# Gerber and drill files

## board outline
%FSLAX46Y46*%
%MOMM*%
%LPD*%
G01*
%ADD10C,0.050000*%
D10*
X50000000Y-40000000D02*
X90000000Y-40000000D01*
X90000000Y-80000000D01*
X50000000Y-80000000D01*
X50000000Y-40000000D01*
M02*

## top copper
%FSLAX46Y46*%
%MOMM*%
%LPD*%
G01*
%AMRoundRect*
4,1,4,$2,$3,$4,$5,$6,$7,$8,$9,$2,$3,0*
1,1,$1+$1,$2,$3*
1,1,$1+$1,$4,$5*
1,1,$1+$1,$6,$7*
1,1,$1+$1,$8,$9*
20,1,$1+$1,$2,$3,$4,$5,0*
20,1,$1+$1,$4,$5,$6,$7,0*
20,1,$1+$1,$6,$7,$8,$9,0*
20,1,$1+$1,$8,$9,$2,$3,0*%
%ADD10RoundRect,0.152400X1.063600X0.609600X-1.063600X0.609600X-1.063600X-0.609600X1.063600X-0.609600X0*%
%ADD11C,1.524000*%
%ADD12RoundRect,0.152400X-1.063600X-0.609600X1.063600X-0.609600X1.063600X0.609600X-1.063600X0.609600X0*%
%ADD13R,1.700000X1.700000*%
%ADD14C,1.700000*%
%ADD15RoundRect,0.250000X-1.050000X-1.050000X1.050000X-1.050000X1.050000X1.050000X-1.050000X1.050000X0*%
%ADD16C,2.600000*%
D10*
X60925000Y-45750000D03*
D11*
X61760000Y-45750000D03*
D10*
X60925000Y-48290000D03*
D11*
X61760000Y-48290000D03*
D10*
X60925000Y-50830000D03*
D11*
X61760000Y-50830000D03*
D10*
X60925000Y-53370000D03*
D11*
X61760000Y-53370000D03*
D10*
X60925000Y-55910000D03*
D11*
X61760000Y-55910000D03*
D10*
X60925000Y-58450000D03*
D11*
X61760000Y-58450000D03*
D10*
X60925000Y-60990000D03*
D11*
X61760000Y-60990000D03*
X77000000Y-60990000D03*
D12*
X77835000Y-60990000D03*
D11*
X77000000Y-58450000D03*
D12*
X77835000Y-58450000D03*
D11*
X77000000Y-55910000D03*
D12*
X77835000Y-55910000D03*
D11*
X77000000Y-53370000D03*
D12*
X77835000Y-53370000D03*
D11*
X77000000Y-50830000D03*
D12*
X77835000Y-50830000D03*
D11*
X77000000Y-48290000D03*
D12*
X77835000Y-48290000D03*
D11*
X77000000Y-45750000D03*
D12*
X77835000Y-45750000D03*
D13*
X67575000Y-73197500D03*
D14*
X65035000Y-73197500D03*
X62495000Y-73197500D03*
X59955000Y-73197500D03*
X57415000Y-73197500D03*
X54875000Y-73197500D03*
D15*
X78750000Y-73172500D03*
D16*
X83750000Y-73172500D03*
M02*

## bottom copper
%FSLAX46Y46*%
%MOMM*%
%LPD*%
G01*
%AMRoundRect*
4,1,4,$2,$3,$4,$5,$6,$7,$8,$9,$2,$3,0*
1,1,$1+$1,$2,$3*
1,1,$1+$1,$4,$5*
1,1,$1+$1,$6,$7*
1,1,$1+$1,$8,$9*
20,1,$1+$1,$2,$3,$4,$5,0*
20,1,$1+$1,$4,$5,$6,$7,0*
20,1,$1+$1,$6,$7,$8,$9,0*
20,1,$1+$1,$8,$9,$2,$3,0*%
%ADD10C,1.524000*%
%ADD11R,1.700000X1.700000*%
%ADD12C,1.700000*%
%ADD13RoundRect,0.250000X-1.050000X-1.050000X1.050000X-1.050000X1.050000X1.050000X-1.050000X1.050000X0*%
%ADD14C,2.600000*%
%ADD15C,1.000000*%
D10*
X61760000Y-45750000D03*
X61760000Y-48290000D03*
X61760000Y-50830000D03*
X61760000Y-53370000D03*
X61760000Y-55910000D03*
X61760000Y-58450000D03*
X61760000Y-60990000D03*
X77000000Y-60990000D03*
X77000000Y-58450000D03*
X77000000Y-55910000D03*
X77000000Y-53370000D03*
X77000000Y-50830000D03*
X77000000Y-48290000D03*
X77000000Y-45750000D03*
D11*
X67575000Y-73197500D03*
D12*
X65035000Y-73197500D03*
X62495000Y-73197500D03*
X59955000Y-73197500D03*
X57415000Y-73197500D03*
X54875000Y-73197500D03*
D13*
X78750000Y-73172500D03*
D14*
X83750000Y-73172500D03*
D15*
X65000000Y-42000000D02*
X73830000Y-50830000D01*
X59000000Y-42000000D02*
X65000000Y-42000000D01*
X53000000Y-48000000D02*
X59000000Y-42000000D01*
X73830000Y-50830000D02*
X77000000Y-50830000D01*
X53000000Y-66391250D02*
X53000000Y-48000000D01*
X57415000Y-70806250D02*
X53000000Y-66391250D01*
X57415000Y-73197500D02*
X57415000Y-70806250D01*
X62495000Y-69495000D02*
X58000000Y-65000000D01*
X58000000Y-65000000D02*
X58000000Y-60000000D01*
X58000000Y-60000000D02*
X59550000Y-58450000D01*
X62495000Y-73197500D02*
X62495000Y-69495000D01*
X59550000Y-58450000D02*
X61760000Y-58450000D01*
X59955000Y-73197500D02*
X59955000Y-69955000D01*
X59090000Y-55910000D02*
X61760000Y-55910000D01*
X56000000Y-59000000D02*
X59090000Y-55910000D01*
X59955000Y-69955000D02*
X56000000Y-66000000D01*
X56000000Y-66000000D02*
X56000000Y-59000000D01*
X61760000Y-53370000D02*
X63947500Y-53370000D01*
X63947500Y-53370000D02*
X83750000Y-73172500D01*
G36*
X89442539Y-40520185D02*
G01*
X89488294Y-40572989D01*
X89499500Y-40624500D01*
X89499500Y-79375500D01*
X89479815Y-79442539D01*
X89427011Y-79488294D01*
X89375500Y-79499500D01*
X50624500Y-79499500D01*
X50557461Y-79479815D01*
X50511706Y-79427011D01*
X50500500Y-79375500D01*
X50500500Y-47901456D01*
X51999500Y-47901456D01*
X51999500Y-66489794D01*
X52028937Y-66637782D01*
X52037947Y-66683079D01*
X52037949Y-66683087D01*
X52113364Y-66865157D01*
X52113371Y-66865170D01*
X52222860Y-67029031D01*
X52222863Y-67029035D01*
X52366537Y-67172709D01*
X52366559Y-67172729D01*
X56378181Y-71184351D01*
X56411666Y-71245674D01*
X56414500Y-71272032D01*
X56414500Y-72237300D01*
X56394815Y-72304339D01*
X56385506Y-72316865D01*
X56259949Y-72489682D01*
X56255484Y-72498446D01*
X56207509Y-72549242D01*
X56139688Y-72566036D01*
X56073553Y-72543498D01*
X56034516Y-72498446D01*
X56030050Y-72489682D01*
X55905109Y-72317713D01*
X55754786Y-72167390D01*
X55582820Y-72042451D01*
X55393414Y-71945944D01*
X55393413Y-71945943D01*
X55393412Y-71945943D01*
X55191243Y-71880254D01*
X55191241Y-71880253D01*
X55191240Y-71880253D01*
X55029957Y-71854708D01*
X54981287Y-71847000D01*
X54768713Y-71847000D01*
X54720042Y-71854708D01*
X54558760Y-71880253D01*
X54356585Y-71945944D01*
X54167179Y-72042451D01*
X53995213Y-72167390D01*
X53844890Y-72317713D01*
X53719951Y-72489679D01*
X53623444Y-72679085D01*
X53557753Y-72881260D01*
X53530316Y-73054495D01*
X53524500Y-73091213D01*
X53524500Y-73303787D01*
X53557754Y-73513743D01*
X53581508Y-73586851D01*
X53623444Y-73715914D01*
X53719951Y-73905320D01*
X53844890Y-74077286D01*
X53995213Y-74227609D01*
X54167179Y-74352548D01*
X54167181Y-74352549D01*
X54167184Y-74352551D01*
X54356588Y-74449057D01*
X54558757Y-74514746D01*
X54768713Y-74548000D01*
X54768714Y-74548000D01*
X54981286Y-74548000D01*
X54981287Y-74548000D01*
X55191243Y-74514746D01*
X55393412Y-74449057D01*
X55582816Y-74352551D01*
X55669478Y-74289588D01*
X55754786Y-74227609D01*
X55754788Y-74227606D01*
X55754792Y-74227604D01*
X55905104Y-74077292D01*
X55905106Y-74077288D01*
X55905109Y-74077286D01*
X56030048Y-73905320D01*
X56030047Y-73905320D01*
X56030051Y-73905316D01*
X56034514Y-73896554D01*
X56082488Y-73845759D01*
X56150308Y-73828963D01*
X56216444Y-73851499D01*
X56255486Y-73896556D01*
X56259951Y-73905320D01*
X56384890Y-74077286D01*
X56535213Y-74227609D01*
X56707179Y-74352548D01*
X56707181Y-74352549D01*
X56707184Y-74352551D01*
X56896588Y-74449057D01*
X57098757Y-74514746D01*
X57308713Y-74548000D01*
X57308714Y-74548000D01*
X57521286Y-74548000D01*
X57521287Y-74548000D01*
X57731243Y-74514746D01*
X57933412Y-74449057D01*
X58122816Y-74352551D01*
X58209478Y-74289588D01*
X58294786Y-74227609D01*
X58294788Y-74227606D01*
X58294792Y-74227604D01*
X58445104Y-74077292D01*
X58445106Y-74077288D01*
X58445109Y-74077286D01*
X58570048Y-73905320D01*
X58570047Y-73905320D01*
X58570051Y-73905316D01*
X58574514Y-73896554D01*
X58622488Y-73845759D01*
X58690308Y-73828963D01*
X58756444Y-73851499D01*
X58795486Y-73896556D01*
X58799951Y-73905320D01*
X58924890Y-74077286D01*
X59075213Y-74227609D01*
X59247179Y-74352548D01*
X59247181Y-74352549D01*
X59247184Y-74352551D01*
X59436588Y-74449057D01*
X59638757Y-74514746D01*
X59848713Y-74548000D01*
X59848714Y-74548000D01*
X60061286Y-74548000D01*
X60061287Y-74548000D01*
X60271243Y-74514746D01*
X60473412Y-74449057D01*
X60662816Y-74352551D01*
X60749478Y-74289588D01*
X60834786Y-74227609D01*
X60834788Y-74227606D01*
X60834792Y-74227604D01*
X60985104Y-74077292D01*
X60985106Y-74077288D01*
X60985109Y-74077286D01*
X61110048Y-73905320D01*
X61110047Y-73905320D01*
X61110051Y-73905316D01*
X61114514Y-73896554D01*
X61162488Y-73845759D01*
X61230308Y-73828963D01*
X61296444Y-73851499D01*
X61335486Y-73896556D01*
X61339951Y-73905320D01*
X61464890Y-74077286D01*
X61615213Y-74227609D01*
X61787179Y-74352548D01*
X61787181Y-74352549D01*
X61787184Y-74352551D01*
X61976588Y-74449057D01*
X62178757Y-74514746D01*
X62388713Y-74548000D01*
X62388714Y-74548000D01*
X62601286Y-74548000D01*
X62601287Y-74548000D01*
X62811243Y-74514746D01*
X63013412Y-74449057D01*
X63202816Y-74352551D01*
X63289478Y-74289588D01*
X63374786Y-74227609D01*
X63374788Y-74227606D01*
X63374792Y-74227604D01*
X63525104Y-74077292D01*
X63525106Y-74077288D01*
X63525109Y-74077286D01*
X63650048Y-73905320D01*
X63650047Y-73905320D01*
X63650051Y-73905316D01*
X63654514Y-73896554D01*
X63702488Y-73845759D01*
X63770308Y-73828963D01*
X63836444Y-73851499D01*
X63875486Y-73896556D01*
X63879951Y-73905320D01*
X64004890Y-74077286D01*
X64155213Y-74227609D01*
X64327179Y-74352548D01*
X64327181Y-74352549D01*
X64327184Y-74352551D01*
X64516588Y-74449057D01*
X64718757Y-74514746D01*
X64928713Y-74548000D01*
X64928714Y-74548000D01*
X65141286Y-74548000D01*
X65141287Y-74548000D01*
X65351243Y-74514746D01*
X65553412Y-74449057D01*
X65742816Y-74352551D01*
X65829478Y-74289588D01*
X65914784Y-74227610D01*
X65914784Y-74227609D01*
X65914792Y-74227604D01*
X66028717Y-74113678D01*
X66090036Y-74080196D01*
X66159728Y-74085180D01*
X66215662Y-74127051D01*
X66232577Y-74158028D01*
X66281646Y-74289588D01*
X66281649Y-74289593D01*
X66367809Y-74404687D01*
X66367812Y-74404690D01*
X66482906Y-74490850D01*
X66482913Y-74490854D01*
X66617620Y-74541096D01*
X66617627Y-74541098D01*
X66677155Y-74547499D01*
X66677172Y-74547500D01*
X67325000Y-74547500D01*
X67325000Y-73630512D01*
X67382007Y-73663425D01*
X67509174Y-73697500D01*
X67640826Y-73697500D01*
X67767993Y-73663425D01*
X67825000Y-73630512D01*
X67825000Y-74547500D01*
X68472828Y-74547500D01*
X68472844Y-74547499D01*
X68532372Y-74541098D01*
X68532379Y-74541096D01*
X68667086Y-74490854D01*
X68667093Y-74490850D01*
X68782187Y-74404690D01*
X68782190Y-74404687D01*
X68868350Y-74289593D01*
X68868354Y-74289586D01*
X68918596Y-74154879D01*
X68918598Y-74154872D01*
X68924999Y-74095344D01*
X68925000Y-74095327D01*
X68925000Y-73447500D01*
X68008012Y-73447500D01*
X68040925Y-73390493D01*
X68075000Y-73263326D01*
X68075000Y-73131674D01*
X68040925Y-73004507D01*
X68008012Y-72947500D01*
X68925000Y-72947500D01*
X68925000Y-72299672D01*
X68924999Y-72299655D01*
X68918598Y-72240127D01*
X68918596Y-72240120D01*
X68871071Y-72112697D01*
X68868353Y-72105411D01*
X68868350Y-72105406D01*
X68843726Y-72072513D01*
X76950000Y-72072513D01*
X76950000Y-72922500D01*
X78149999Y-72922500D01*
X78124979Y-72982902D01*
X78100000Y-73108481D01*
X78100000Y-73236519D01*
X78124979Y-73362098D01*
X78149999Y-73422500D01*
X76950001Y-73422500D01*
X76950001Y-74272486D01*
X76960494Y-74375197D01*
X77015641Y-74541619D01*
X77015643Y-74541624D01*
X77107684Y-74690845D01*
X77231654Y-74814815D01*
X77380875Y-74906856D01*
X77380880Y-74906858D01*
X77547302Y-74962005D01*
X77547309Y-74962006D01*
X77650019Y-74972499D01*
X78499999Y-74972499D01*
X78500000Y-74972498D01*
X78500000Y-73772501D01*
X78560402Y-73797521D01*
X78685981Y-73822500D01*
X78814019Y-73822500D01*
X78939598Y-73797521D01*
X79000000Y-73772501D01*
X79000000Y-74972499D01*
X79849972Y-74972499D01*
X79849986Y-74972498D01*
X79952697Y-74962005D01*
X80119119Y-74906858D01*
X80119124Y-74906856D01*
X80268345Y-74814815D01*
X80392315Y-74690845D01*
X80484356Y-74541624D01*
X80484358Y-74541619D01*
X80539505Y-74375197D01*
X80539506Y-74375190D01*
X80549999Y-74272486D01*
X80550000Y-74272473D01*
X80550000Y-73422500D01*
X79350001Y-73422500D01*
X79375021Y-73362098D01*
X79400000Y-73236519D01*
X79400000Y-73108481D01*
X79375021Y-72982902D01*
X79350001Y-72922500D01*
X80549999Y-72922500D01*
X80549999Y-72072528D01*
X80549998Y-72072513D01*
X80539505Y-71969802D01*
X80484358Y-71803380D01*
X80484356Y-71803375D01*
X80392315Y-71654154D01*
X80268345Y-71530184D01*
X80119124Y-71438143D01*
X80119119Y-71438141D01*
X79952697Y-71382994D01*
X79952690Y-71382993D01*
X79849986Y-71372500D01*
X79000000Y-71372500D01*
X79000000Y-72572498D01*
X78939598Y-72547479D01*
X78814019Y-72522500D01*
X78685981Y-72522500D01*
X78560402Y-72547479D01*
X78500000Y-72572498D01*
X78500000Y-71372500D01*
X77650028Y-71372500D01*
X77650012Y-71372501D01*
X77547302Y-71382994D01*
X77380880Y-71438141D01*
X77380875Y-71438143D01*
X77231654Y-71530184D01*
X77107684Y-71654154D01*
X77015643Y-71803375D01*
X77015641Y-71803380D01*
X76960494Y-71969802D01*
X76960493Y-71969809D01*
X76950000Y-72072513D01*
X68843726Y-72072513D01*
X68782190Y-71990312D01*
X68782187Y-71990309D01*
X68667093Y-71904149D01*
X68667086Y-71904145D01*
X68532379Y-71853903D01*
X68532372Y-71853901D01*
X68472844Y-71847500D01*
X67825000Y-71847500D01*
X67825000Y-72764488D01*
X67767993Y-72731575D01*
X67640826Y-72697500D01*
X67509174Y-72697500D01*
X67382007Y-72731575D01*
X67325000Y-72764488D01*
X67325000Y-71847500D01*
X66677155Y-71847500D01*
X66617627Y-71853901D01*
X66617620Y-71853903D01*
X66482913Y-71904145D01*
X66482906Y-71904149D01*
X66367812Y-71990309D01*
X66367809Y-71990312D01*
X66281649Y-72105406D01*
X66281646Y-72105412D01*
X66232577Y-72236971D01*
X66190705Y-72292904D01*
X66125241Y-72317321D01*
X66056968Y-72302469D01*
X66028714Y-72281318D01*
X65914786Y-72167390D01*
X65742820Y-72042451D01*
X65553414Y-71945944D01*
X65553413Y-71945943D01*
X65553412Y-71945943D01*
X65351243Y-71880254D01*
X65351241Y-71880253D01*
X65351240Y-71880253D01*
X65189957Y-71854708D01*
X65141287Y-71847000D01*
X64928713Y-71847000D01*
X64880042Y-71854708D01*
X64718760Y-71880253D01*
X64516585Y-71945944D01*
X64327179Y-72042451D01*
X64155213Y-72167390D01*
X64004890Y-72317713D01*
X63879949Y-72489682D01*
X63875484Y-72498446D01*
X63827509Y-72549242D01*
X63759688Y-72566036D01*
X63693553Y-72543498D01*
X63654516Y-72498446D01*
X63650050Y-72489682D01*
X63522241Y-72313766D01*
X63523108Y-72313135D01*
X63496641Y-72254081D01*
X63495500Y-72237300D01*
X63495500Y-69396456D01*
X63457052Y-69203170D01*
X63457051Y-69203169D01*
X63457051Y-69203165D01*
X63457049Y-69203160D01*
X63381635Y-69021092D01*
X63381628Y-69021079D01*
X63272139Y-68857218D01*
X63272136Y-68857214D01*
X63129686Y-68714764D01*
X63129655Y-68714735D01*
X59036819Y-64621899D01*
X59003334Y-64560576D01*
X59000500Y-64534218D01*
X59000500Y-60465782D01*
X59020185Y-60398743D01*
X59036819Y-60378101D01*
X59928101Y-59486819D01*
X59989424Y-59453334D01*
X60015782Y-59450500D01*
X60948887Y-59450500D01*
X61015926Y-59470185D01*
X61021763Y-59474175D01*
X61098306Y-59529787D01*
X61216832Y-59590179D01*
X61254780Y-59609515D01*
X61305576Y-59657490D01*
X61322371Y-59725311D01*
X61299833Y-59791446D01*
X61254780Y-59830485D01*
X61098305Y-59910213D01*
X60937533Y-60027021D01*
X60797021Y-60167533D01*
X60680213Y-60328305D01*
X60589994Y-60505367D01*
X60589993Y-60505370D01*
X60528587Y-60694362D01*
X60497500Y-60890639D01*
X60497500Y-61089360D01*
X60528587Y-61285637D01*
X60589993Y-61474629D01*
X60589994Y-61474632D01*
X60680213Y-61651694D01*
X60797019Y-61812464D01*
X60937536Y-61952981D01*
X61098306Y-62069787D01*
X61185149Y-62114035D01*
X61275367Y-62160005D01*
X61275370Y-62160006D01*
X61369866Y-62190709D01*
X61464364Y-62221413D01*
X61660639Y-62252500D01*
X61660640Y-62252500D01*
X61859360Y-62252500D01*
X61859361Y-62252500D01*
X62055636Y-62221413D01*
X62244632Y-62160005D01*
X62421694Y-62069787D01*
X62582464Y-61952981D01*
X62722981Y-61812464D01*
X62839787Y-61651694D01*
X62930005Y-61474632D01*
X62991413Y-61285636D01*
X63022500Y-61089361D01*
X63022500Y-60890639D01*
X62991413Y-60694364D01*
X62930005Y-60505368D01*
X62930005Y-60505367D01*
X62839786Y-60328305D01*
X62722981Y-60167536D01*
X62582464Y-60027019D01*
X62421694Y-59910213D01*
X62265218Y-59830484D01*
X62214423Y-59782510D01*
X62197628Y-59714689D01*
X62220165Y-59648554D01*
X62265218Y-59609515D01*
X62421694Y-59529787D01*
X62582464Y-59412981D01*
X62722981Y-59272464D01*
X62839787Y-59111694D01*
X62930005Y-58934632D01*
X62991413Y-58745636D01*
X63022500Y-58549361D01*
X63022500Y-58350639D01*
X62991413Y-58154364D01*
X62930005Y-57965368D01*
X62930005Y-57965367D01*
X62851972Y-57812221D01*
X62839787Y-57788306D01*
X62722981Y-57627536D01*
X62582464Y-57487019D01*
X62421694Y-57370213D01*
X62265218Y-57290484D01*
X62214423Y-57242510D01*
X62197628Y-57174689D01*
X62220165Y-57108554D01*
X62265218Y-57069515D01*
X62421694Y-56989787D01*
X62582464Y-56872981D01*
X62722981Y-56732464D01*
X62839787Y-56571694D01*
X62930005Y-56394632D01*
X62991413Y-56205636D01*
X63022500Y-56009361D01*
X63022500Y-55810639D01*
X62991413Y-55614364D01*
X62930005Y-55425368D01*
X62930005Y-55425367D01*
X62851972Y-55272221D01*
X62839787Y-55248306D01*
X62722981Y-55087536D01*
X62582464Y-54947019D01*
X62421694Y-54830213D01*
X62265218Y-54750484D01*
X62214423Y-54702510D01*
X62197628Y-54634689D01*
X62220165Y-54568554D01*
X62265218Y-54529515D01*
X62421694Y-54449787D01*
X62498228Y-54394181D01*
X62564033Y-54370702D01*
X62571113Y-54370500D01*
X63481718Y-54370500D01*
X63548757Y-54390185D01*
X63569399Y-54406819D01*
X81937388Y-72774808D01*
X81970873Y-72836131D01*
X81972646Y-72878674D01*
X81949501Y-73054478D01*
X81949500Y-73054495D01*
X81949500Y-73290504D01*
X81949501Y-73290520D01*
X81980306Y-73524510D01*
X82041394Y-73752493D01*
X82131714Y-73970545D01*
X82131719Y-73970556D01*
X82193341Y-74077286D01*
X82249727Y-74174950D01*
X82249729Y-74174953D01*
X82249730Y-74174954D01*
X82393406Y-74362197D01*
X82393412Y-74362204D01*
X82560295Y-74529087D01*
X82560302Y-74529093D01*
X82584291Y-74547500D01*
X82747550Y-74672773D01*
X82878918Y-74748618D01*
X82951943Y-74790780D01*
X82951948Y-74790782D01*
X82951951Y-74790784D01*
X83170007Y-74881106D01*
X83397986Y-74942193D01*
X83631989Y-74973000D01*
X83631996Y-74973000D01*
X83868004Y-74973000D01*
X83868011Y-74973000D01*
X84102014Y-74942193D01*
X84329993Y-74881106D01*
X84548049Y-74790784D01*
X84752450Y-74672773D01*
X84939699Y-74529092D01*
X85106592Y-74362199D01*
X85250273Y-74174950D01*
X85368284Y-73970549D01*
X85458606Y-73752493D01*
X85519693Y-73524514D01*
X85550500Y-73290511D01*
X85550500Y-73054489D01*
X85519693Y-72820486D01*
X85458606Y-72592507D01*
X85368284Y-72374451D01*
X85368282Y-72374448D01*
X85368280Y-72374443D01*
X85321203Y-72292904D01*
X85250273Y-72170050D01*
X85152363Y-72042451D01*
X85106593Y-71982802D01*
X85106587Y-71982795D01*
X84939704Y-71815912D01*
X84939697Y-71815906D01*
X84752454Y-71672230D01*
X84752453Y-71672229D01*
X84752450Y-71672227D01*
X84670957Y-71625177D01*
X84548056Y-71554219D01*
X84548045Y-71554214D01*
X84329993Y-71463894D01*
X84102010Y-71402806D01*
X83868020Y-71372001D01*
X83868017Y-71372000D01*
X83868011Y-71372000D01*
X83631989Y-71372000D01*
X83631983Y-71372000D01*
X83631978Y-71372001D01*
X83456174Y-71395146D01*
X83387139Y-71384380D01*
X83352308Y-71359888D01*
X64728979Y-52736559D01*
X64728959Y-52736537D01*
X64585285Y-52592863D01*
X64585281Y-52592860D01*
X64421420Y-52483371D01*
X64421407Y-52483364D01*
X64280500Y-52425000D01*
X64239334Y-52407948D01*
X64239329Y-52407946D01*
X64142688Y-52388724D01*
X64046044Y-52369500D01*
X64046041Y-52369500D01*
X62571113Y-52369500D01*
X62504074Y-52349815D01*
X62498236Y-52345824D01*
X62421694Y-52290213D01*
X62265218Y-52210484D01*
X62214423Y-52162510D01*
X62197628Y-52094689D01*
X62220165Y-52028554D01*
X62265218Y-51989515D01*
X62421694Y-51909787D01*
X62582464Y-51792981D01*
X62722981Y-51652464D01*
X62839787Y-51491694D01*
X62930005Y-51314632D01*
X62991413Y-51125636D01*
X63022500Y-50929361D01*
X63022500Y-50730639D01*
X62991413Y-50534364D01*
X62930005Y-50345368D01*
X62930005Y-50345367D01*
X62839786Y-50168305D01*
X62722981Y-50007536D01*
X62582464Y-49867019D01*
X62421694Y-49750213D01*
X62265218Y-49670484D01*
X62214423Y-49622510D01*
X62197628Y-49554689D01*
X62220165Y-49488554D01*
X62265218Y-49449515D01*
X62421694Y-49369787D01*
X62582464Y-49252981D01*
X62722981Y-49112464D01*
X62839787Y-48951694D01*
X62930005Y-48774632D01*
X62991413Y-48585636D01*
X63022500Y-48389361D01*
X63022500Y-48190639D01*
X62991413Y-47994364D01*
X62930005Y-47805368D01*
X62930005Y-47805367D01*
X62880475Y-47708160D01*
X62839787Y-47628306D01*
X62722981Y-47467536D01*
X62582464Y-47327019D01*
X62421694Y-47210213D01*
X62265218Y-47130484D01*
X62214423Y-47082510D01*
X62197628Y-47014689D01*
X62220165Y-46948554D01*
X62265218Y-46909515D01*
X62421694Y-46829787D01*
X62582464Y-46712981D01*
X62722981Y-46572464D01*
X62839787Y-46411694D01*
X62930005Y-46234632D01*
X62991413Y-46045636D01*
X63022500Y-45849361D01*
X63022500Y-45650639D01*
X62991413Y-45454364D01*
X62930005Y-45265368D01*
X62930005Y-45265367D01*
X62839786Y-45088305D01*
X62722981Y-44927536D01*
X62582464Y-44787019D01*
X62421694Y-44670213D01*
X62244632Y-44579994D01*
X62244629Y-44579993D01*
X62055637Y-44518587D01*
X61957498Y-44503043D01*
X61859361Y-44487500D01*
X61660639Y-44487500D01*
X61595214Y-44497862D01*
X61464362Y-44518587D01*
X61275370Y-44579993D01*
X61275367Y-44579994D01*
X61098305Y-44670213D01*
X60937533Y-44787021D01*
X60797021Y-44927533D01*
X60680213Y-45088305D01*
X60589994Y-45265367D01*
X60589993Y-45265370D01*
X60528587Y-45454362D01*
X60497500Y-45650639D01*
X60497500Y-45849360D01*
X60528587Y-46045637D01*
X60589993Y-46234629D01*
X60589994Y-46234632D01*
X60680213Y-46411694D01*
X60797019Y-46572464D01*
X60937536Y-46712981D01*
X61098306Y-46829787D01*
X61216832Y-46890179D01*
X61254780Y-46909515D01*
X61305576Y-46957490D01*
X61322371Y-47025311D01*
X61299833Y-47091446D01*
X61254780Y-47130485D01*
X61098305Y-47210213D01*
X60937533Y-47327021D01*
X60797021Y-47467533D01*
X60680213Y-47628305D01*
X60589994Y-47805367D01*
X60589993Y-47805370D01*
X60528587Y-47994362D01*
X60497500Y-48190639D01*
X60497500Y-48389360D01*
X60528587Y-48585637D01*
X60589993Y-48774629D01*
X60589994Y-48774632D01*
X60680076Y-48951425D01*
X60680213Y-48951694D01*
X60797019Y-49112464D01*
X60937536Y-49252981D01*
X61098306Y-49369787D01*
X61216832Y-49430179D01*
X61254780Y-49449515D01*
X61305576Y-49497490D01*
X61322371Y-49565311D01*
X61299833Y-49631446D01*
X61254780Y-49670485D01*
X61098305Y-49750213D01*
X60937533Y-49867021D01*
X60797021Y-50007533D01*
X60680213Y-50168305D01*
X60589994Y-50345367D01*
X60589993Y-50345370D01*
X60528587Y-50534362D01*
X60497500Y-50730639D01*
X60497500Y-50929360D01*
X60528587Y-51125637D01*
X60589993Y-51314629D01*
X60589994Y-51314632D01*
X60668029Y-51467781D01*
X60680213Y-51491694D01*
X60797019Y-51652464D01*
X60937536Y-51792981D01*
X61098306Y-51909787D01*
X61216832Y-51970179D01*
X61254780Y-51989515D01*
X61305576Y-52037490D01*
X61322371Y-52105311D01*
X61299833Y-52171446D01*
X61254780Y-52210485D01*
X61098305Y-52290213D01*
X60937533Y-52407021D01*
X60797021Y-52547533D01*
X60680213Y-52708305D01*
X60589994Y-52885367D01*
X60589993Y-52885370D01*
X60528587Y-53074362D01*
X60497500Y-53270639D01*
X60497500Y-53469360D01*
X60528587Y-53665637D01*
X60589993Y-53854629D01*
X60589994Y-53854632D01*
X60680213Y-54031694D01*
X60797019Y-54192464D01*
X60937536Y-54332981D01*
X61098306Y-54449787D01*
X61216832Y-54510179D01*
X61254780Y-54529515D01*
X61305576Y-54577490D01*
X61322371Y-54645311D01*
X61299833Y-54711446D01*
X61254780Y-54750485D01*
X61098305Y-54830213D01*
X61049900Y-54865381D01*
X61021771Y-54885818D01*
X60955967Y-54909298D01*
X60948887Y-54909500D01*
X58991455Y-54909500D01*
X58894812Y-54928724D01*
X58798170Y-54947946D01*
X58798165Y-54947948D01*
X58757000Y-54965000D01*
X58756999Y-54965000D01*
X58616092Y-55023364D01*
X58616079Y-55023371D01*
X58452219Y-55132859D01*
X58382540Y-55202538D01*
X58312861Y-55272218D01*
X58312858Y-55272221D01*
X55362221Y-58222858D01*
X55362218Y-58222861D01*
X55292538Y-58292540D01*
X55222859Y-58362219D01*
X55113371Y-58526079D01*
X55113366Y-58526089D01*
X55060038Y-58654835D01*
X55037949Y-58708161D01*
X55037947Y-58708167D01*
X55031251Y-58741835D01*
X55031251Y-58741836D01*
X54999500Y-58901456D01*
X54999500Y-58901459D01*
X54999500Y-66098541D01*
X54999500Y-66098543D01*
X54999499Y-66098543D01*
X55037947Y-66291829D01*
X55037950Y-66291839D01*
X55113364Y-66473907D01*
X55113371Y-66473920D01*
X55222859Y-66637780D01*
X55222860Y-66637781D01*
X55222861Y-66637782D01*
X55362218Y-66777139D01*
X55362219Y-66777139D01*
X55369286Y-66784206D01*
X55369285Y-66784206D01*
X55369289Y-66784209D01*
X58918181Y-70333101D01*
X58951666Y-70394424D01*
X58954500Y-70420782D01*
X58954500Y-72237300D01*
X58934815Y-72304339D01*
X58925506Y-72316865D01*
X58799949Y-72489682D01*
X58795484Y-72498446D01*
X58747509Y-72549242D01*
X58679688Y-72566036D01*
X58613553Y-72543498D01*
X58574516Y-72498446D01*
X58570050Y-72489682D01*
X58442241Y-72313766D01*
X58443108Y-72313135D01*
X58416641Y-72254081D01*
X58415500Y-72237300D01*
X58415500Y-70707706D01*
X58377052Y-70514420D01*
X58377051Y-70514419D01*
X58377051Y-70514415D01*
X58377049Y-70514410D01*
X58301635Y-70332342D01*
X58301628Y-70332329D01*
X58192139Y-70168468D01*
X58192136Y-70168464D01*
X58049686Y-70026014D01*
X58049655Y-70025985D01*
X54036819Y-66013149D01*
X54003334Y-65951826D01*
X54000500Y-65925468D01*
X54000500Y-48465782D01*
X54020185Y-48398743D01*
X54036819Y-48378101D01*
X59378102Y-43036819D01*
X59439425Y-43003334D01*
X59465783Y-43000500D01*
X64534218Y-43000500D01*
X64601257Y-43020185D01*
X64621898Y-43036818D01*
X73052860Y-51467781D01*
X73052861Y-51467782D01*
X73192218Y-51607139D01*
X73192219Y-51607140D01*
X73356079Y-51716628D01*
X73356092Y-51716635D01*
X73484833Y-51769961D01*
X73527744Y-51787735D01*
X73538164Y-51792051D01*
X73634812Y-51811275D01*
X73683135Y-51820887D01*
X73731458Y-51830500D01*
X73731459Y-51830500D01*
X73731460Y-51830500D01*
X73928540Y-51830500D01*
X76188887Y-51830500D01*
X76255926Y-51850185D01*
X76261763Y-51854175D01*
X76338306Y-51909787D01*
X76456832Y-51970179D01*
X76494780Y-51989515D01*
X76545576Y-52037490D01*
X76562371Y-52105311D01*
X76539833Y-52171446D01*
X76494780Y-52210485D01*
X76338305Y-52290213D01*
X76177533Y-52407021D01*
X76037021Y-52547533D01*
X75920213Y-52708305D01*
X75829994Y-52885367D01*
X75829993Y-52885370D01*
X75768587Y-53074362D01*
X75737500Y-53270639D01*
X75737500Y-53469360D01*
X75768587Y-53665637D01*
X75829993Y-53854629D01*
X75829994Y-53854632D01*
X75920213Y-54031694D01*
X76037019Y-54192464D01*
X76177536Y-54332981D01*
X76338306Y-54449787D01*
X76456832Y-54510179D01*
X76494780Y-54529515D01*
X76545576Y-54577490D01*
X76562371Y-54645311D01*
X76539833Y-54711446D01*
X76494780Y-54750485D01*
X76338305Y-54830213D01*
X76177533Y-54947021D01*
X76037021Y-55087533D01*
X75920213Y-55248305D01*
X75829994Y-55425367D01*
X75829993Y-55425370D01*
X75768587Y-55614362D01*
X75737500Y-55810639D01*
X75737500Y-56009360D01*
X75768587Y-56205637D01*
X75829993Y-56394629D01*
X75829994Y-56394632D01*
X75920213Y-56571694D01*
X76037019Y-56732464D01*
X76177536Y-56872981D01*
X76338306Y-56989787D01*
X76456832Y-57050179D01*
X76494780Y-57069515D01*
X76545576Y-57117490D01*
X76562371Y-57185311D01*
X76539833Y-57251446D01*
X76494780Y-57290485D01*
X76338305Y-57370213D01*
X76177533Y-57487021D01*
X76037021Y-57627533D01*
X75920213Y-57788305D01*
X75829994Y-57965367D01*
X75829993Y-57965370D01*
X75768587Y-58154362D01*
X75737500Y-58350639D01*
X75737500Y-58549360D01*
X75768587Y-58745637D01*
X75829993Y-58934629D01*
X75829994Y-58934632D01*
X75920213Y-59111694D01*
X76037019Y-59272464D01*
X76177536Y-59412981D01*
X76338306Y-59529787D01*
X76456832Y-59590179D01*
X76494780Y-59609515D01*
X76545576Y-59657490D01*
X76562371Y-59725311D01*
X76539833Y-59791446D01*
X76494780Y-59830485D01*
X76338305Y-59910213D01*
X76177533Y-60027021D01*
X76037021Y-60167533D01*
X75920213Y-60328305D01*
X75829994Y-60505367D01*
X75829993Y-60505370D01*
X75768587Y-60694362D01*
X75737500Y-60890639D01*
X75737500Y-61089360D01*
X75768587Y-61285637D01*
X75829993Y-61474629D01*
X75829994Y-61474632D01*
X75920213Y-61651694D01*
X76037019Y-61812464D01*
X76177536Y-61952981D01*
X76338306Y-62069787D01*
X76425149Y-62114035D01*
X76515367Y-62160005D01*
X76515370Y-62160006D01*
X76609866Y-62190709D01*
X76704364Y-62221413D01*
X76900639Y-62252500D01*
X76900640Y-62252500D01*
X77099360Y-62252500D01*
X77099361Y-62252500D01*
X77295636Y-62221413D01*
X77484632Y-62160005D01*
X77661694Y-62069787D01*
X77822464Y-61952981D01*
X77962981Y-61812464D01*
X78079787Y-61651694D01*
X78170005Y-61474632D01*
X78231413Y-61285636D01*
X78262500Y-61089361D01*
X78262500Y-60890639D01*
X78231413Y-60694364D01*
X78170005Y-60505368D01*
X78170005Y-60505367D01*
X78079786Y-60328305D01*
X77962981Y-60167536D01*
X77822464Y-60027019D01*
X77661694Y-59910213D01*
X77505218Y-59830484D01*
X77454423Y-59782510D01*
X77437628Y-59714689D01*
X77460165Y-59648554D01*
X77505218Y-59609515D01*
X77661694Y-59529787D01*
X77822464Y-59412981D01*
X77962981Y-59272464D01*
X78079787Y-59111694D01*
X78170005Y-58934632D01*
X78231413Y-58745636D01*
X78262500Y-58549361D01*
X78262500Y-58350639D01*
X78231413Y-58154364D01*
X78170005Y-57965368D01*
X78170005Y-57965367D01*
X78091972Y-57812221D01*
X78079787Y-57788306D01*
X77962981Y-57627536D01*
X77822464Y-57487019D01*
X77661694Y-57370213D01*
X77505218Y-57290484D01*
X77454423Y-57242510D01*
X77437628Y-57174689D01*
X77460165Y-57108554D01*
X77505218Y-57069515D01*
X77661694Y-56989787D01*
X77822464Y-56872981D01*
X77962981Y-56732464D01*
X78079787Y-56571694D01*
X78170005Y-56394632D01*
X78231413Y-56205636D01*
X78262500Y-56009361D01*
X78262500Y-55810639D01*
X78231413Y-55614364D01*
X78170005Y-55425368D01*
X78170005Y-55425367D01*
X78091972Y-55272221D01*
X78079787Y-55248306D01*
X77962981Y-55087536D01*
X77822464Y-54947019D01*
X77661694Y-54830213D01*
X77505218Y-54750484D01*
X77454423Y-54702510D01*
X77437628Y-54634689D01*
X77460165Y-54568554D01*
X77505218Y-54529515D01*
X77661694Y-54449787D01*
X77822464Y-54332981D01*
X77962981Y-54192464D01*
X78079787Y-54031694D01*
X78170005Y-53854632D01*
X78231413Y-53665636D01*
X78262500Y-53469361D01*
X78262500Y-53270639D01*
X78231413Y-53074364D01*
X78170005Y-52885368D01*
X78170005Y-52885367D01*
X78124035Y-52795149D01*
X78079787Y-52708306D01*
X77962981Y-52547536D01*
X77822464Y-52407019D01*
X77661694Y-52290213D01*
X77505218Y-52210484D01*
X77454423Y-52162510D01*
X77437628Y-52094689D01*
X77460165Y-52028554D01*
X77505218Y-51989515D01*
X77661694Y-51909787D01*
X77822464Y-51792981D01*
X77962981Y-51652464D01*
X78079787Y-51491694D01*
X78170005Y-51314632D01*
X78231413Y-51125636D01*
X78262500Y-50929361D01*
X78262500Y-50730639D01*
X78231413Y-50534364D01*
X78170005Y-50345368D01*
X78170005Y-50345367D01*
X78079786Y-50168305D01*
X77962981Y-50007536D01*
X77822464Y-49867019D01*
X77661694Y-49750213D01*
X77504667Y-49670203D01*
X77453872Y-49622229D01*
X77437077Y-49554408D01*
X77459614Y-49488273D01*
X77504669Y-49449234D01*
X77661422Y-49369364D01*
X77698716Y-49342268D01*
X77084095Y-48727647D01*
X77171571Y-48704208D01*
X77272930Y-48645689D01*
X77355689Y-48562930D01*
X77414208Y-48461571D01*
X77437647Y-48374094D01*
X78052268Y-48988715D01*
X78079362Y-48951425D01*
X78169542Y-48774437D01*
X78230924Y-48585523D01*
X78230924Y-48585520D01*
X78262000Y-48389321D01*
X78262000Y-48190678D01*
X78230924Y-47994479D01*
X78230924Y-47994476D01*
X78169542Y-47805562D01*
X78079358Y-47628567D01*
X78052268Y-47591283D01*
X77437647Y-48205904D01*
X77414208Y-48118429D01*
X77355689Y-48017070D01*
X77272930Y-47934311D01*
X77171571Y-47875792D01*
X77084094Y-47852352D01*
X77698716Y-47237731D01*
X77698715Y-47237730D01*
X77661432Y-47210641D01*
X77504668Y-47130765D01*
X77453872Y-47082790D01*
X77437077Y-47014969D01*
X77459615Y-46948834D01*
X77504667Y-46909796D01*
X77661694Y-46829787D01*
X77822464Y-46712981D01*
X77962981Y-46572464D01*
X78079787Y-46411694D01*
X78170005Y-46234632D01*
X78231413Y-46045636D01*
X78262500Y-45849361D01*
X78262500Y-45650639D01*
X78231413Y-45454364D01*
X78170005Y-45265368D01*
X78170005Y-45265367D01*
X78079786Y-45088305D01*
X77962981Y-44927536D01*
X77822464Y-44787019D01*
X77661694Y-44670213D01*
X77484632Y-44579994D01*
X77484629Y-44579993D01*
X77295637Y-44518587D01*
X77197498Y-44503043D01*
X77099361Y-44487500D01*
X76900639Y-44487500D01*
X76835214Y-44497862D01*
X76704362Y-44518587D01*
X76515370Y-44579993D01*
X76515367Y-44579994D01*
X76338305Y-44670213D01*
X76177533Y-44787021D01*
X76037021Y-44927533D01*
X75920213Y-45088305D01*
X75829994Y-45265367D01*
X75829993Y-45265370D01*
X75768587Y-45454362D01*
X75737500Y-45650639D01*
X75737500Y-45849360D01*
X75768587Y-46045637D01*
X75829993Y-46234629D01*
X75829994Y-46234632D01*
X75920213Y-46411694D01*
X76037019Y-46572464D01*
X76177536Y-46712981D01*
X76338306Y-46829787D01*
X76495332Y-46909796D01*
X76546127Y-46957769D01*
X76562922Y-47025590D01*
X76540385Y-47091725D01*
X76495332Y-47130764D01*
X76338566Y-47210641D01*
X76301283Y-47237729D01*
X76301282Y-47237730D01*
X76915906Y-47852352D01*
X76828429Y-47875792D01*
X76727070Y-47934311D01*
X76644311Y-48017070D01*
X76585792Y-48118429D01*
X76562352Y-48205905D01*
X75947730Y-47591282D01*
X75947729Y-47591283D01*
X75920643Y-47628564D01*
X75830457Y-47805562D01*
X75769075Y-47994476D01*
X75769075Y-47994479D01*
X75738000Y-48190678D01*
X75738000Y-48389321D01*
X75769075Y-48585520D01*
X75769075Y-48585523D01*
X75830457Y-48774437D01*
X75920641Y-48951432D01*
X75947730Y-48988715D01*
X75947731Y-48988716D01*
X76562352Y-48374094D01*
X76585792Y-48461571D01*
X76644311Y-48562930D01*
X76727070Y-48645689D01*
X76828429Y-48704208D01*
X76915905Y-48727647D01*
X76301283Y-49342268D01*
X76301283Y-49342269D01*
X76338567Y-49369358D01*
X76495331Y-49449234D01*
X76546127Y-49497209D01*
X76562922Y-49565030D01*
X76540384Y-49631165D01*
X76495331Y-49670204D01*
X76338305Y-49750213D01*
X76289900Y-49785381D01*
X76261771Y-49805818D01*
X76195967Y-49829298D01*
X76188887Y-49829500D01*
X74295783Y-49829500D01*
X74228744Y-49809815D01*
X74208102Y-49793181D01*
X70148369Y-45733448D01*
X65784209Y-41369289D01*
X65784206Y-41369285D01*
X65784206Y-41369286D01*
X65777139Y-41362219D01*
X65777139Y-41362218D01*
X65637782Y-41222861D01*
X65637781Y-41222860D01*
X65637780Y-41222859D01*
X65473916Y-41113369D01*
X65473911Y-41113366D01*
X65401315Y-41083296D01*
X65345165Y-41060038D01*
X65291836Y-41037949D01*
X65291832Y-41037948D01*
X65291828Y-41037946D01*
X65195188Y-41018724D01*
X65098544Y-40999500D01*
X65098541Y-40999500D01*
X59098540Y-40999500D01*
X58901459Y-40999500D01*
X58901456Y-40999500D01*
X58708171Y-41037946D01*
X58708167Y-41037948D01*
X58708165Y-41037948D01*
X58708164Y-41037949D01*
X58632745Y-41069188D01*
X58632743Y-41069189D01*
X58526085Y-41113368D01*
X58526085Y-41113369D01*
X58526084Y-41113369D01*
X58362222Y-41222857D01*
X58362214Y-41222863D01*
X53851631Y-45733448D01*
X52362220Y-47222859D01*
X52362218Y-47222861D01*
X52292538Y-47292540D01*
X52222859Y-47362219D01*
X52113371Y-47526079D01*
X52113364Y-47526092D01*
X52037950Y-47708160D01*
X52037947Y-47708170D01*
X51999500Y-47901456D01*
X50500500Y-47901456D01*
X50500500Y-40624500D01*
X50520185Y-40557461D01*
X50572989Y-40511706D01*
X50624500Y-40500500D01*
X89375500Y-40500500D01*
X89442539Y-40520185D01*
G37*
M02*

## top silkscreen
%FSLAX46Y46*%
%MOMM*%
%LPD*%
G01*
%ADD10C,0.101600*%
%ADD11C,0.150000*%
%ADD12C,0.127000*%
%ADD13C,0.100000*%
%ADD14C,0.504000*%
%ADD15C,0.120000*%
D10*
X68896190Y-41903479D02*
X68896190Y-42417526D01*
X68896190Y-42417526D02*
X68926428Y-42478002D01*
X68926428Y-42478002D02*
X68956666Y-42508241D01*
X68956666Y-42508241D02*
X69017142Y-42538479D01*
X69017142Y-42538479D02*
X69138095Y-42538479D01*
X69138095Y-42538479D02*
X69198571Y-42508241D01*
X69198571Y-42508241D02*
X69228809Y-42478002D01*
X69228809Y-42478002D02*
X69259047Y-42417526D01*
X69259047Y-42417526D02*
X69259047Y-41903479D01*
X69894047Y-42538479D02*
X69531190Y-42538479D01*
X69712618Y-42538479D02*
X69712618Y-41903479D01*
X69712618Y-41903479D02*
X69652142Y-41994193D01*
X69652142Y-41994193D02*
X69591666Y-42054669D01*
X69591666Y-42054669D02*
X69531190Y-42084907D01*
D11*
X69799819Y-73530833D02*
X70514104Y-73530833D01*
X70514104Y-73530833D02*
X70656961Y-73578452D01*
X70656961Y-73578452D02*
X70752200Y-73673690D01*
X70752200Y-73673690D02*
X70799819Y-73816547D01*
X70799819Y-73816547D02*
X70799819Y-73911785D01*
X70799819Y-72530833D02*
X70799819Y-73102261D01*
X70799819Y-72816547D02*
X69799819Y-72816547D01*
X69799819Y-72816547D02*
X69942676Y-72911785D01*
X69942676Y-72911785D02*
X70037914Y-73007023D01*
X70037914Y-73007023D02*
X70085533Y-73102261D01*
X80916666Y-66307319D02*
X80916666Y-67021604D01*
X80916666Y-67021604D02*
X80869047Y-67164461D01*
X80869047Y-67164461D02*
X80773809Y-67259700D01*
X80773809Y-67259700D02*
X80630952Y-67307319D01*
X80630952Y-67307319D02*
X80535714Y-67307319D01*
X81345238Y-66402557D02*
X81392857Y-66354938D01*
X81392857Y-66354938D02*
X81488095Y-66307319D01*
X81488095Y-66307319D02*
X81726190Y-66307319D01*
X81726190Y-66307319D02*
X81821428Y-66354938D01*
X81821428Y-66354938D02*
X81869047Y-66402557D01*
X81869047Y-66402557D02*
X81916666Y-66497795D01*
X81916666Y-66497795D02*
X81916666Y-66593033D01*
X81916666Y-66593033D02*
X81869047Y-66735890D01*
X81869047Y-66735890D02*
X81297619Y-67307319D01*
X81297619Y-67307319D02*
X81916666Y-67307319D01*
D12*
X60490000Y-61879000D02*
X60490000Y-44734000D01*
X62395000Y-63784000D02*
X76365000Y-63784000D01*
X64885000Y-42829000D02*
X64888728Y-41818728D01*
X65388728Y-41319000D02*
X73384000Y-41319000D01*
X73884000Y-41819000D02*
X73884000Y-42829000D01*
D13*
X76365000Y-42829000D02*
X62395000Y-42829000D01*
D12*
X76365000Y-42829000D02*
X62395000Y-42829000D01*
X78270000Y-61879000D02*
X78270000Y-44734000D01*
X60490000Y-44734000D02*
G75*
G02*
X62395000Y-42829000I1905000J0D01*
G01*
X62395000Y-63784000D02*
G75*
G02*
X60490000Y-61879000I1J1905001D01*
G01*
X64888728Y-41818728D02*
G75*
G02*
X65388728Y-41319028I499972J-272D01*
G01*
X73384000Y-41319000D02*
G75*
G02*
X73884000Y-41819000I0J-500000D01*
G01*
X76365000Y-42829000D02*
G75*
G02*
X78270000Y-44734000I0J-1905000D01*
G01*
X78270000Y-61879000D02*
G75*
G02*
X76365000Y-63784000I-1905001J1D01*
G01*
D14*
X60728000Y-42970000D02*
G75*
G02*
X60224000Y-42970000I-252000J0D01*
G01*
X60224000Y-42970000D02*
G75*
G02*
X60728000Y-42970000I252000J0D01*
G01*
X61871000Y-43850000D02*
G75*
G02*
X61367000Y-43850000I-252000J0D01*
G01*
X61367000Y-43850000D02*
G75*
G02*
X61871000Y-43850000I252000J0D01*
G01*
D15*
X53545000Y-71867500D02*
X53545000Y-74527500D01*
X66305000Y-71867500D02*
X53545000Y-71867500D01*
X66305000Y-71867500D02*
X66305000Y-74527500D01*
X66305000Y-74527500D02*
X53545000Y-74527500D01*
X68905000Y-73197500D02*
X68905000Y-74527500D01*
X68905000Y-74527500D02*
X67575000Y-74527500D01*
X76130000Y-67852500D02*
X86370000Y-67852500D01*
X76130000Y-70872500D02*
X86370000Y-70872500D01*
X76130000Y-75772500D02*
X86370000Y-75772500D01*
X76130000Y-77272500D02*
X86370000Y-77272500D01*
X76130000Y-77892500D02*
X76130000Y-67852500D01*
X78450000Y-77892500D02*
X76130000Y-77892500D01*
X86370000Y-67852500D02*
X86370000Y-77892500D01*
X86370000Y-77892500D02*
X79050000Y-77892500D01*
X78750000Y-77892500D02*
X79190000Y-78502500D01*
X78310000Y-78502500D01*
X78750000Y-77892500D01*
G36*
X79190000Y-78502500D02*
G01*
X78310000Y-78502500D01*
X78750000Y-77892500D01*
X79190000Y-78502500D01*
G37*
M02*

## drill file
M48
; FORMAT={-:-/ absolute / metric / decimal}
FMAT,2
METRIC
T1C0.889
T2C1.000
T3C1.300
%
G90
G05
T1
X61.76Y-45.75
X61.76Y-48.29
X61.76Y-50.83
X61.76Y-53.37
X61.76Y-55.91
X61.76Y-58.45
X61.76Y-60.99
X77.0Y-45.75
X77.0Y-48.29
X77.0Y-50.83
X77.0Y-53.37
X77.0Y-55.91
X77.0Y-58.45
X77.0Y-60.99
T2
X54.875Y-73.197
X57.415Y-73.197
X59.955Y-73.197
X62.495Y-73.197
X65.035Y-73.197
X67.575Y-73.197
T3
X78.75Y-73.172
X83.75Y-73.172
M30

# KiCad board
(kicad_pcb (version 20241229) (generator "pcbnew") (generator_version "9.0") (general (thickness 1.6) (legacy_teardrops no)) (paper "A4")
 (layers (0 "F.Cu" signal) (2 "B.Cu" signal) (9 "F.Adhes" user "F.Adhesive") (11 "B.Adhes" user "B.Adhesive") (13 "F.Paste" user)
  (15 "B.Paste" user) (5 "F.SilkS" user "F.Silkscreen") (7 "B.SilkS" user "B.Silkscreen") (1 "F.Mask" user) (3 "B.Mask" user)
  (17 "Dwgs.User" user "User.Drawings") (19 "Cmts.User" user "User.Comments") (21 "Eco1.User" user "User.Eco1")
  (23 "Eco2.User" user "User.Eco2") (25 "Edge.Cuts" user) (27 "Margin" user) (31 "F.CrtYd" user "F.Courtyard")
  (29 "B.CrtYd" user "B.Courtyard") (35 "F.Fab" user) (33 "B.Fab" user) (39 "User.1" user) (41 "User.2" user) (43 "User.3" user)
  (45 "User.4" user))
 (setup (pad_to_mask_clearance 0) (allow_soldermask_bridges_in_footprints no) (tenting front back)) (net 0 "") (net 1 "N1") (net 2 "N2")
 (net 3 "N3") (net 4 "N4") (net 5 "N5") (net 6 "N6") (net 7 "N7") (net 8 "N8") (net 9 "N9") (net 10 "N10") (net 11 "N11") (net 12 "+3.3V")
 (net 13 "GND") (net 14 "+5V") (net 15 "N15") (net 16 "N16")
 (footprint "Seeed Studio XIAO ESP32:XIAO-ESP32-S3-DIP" (layer "F.Cu") (at 69.38 53.37 90)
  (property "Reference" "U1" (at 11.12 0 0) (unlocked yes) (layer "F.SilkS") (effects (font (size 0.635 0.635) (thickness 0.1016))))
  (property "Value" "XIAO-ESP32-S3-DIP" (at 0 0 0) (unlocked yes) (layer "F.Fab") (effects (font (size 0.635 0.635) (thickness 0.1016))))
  (fp_line (start -8.509 -8.89) (end 8.636 -8.89) (stroke (width 0.127) (type solid)) (layer "F.SilkS"))
  (fp_line (start -10.414 -6.985) (end -10.414 6.985) (stroke (width 0.127) (type solid)) (layer "F.SilkS"))
  (fp_line (start 10.541 -4.495) (end 11.551272 -4.491272) (stroke (width 0.127) (type solid)) (layer "F.SilkS"))
  (fp_line (start 12.051 -3.991272) (end 12.051 4.004) (stroke (width 0.127) (type solid)) (layer "F.SilkS"))
  (fp_line (start 11.551 4.504) (end 10.541 4.504) (stroke (width 0.127) (type solid)) (layer "F.SilkS"))
  (fp_line (start 10.541 6.985) (end 10.541 -6.985) (stroke (width 0.1) (type solid)) (layer "F.SilkS"))
  (fp_line (start 10.541 6.985) (end 10.541 -6.985) (stroke (width 0.127) (type solid)) (layer "F.SilkS"))
  (fp_line (start -8.509 8.89) (end 8.636 8.89) (stroke (width 0.127) (type solid)) (layer "F.SilkS"))
  (fp_arc (start 8.636 -8.89) (mid 9.983038 -8.332038) (end 10.541 -6.985) (stroke (width 0.127) (type solid)) (layer "F.SilkS"))
  (fp_arc (start -10.414 -6.985) (mid -9.856038 -8.332038) (end -8.509 -8.89) (stroke (width 0.127) (type solid)) (layer "F.SilkS"))
  (fp_arc (start 11.551272 -4.491272) (mid 11.904644 -4.344724) (end 12.051 -3.991272) (stroke (width 0.127) (type default))
   (layer "F.SilkS"))
  (fp_arc (start 12.051 4.004) (mid 11.904553 4.357553) (end 11.551 4.504) (stroke (width 0.127) (type default)) (layer "F.SilkS"))
  (fp_arc (start 10.541 6.985) (mid 9.983038 8.332038) (end 8.636 8.89) (stroke (width 0.127) (type solid)) (layer "F.SilkS"))
  (fp_arc (start -8.509 8.89) (mid -9.856038 8.332038) (end -10.414 6.985) (stroke (width 0.127) (type solid)) (layer "F.SilkS"))
  (fp_circle (center 10.4 -8.904) (end 10.654 -8.904) (stroke (width 0.5) (type solid)) (fill yes) (layer "F.SilkS"))
  (fp_circle (center 9.52 -7.761) (end 9.774 -7.761) (stroke (width 0.5) (type solid)) (fill yes) (layer "F.SilkS"))
  (pad "1" smd roundrect (at 7.62 -8.455 180) (size 2.432 1.524) (layers "F.Cu" "F.Mask") (roundrect_rratio 0.1) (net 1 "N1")
   (thermal_bridge_angle 45))
  (pad "1" thru_hole circle (at 7.62 -7.62 180) (size 1.524 1.524) (drill 0.889) (layers "*.Cu" "*.Mask") (remove_unused_layers no)
   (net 1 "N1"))
  (pad "2" smd roundrect (at 5.08 -8.455 180) (size 2.432 1.524) (layers "F.Cu" "F.Mask") (roundrect_rratio 0.1) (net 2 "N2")
   (thermal_bridge_angle 45))
  (pad "2" thru_hole circle (at 5.08 -7.62 180) (size 1.524 1.524) (drill 0.889) (layers "*.Cu" "*.Mask") (remove_unused_layers no)
   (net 2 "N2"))
  (pad "3" smd roundrect (at 2.54 -8.455 180) (size 2.432 1.524) (layers "F.Cu" "F.Mask") (roundrect_rratio 0.1) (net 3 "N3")
   (thermal_bridge_angle 45))
  (pad "3" thru_hole circle (at 2.54 -7.62 180) (size 1.524 1.524) (drill 0.889) (layers "*.Cu" "*.Mask") (remove_unused_layers no)
   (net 3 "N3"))
  (pad "4" smd roundrect (at 0 -8.455 180) (size 2.432 1.524) (layers "F.Cu" "F.Mask") (roundrect_rratio 0.1) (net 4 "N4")
   (thermal_bridge_angle 45))
  (pad "4" thru_hole circle (at 0 -7.62 180) (size 1.524 1.524) (drill 0.889) (layers "*.Cu" "*.Mask") (remove_unused_layers no)
   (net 4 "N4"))
  (pad "5" smd roundrect (at -2.54 -8.455 180) (size 2.432 1.524) (layers "F.Cu" "F.Mask") (roundrect_rratio 0.1) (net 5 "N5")
   (thermal_bridge_angle 45))
  (pad "5" thru_hole circle (at -2.54 -7.62 180) (size 1.524 1.524) (drill 0.889) (layers "*.Cu" "*.Mask") (remove_unused_layers no)
   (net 5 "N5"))
  (pad "6" smd roundrect (at -5.08 -8.455 180) (size 2.432 1.524) (layers "F.Cu" "F.Mask") (roundrect_rratio 0.1) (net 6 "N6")
   (thermal_bridge_angle 45))
  (pad "6" thru_hole circle (at -5.08 -7.62 180) (size 1.524 1.524) (drill 0.889) (layers "*.Cu" "*.Mask") (remove_unused_layers no)
   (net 6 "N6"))
  (pad "7" smd roundrect (at -7.62 -8.455 180) (size 2.432 1.524) (layers "F.Cu" "F.Mask") (roundrect_rratio 0.1) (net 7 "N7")
   (thermal_bridge_angle 45))
  (pad "7" thru_hole circle (at -7.62 -7.62 180) (size 1.524 1.524) (drill 0.889) (layers "*.Cu" "*.Mask") (remove_unused_layers no)
   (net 7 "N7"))
  (pad "8" thru_hole circle (at -7.62 7.62) (size 1.524 1.524) (drill 0.889) (layers "*.Cu" "*.Mask") (remove_unused_layers no) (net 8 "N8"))
  (pad "8" smd roundrect (at -7.62 8.455) (size 2.432 1.524) (layers "F.Cu" "F.Mask") (roundrect_rratio 0.1) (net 8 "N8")
   (thermal_bridge_angle 45))
  (pad "9" thru_hole circle (at -5.08 7.62) (size 1.524 1.524) (drill 0.889) (layers "*.Cu" "*.Mask") (remove_unused_layers no) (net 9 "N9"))
  (pad "9" smd roundrect (at -5.08 8.455) (size 2.432 1.524) (layers "F.Cu" "F.Mask") (roundrect_rratio 0.1) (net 9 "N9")
   (thermal_bridge_angle 45))
  (pad "10" thru_hole circle (at -2.54 7.62) (size 1.524 1.524) (drill 0.889) (layers "*.Cu" "*.Mask") (remove_unused_layers no)
   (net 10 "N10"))
  (pad "10" smd roundrect (at -2.54 8.455) (size 2.432 1.524) (layers "F.Cu" "F.Mask") (roundrect_rratio 0.1) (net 10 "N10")
   (thermal_bridge_angle 45))
  (pad "11" thru_hole circle (at 0 7.62) (size 1.524 1.524) (drill 0.889) (layers "*.Cu" "*.Mask") (remove_unused_layers no) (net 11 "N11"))
  (pad "11" smd roundrect (at 0 8.455) (size 2.432 1.524) (layers "F.Cu" "F.Mask") (roundrect_rratio 0.1) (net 11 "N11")
   (thermal_bridge_angle 45))
  (pad "12" thru_hole circle (at 2.54 7.62) (size 1.524 1.524) (drill 0.889) (layers "*.Cu" "*.Mask") (remove_unused_layers no)
   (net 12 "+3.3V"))
  (pad "12" smd roundrect (at 2.54 8.455) (size 2.432 1.524) (layers "F.Cu" "F.Mask") (roundrect_rratio 0.1) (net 12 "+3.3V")
   (thermal_bridge_angle 45))
  (pad "13" thru_hole circle (at 5.08 7.62) (size 1.524 1.524) (drill 0.889) (layers "*.Cu" "*.Mask") (remove_unused_layers no)
   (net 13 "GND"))
  (pad "13" smd roundrect (at 5.08 8.455) (size 2.432 1.524) (layers "F.Cu" "F.Mask") (roundrect_rratio 0.1) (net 13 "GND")
   (thermal_bridge_angle 45))
  (pad "14" thru_hole circle (at 7.62 7.62) (size 1.524 1.524) (drill 0.889) (layers "*.Cu" "*.Mask") (remove_unused_layers no)
   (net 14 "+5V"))
  (pad "14" smd roundrect (at 7.62 8.455) (size 2.432 1.524) (layers "F.Cu" "F.Mask") (roundrect_rratio 0.1) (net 14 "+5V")
   (thermal_bridge_angle 45)))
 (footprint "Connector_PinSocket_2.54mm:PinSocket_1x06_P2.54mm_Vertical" (layer "F.Cu") (at 67.575 73.1975 -90)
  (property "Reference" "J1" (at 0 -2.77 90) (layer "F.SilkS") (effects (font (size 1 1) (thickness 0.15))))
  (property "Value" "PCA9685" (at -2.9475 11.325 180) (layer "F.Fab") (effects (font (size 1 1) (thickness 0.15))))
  (fp_line (start -1.33 14.03) (end 1.33 14.03) (stroke (width 0.12) (type solid)) (layer "F.SilkS"))
  (fp_line (start -1.33 1.27) (end -1.33 14.03) (stroke (width 0.12) (type solid)) (layer "F.SilkS"))
  (fp_line (start -1.33 1.27) (end 1.33 1.27) (stroke (width 0.12) (type solid)) (layer "F.SilkS"))
  (fp_line (start 1.33 1.27) (end 1.33 14.03) (stroke (width 0.12) (type solid)) (layer "F.SilkS"))
  (fp_line (start 0 -1.33) (end 1.33 -1.33) (stroke (width 0.12) (type solid)) (layer "F.SilkS"))
  (fp_line (start 1.33 -1.33) (end 1.33 0) (stroke (width 0.12) (type solid)) (layer "F.SilkS"))
  (pad "1" thru_hole rect (at 0 0 270) (size 1.7 1.7) (drill 1) (layers "*.Cu" "*.Mask") (remove_unused_layers no) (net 13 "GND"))
  (pad "2" thru_hole circle (at 0 2.54 270) (size 1.7 1.7) (drill 1) (layers "*.Cu" "*.Mask") (remove_unused_layers no) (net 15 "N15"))
  (pad "3" thru_hole circle (at 0 5.08 270) (size 1.7 1.7) (drill 1) (layers "*.Cu" "*.Mask") (remove_unused_layers no) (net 6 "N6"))
  (pad "4" thru_hole circle (at 0 7.62 270) (size 1.7 1.7) (drill 1) (layers "*.Cu" "*.Mask") (remove_unused_layers no) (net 5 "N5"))
  (pad "5" thru_hole circle (at 0 10.16 270) (size 1.7 1.7) (drill 1) (layers "*.Cu" "*.Mask") (remove_unused_layers no) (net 12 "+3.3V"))
  (pad "6" thru_hole circle (at 0 12.7 270) (size 1.7 1.7) (drill 1) (layers "*.Cu" "*.Mask") (remove_unused_layers no) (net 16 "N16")))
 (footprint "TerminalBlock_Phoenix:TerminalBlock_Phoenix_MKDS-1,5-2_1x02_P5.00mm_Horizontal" (layer "F.Cu") (at 78.75 73.1725)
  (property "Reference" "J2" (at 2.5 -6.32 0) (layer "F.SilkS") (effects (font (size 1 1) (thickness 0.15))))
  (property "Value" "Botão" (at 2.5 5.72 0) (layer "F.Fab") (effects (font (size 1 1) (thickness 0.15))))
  (fp_line (start -2.62 -5.32) (end 7.62 -5.32) (stroke (width 0.12) (type solid)) (layer "F.SilkS"))
  (fp_line (start -2.62 -2.3) (end 7.62 -2.3) (stroke (width 0.12) (type solid)) (layer "F.SilkS"))
  (fp_line (start -2.62 2.6) (end 7.62 2.6) (stroke (width 0.12) (type solid)) (layer "F.SilkS"))
  (fp_line (start -2.62 4.1) (end 7.62 4.1) (stroke (width 0.12) (type solid)) (layer "F.SilkS"))
  (fp_line (start -2.62 4.72) (end -2.62 -5.32) (stroke (width 0.12) (type solid)) (layer "F.SilkS"))
  (fp_line (start -0.3 4.72) (end -2.62 4.72) (stroke (width 0.12) (type solid)) (layer "F.SilkS"))
  (fp_line (start 7.62 -5.32) (end 7.62 4.72) (stroke (width 0.12) (type solid)) (layer "F.SilkS"))
  (fp_line (start 7.62 4.72) (end 0.3 4.72) (stroke (width 0.12) (type solid)) (layer "F.SilkS"))
  (fp_poly (pts (xy 0 4.72) (xy 0.44 5.33) (xy -0.44 5.33)) (stroke (width 0.12) (type solid)) (fill yes) (layer "F.SilkS"))
  (pad "1" thru_hole roundrect (at 0 0) (size 2.6 2.6) (drill 1.3) (layers "*.Cu" "*.Mask") (remove_unused_layers no)
   (roundrect_rratio 0.096154) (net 13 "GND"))
  (pad "2" thru_hole circle (at 5 0) (size 2.6 2.6) (drill 1.3) (layers "*.Cu" "*.Mask") (remove_unused_layers no) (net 4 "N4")))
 (gr_rect (start 50 40) (end 90 80) (stroke (width 0.05) (type default)) (fill no) (layer "Edge.Cuts"))
 (segment (start 65 42) (end 73.83 50.83) (width 1) (layer "B.Cu") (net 12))
 (segment (start 59 42) (end 65 42) (width 1) (layer "B.Cu") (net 12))
 (segment (start 53 48) (end 59 42) (width 1) (layer "B.Cu") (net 12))
 (segment (start 73.83 50.83) (end 77 50.83) (width 1) (layer "B.Cu") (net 12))
 (segment (start 53 66.39125) (end 53 48) (width 1) (layer "B.Cu") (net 12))
 (segment (start 57.415 70.80625) (end 53 66.39125) (width 1) (layer "B.Cu") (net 12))
 (segment (start 57.415 73.1975) (end 57.415 70.80625) (width 1) (layer "B.Cu") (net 12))
 (segment (start 62.495 69.495) (end 58 65) (width 1) (layer "B.Cu") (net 6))
 (segment (start 58 65) (end 58 60) (width 1) (layer "B.Cu") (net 6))
 (segment (start 58 60) (end 59.55 58.45) (width 1) (layer "B.Cu") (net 6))
 (segment (start 62.495 73.1975) (end 62.495 69.495) (width 1) (layer "B.Cu") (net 6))
 (segment (start 59.55 58.45) (end 61.76 58.45) (width 1) (layer "B.Cu") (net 6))
 (segment (start 59.955 73.1975) (end 59.955 69.955) (width 1) (layer "B.Cu") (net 5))
 (segment (start 59.09 55.91) (end 61.76 55.91) (width 1) (layer "B.Cu") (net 5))
 (segment (start 56 59) (end 59.09 55.91) (width 1) (layer "B.Cu") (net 5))
 (segment (start 59.955 69.955) (end 56 66) (width 1) (layer "B.Cu") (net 5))
 (segment (start 56 66) (end 56 59) (width 1) (layer "B.Cu") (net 5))
 (segment (start 61.76 53.37) (end 63.9475 53.37) (width 1) (layer "B.Cu") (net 4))
 (segment (start 63.9475 53.37) (end 83.75 73.1725) (width 1) (layer "B.Cu") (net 4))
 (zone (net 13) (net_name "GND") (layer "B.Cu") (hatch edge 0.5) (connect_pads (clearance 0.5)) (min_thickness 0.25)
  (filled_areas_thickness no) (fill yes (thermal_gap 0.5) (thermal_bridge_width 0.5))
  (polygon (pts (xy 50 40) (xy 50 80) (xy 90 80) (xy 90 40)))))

